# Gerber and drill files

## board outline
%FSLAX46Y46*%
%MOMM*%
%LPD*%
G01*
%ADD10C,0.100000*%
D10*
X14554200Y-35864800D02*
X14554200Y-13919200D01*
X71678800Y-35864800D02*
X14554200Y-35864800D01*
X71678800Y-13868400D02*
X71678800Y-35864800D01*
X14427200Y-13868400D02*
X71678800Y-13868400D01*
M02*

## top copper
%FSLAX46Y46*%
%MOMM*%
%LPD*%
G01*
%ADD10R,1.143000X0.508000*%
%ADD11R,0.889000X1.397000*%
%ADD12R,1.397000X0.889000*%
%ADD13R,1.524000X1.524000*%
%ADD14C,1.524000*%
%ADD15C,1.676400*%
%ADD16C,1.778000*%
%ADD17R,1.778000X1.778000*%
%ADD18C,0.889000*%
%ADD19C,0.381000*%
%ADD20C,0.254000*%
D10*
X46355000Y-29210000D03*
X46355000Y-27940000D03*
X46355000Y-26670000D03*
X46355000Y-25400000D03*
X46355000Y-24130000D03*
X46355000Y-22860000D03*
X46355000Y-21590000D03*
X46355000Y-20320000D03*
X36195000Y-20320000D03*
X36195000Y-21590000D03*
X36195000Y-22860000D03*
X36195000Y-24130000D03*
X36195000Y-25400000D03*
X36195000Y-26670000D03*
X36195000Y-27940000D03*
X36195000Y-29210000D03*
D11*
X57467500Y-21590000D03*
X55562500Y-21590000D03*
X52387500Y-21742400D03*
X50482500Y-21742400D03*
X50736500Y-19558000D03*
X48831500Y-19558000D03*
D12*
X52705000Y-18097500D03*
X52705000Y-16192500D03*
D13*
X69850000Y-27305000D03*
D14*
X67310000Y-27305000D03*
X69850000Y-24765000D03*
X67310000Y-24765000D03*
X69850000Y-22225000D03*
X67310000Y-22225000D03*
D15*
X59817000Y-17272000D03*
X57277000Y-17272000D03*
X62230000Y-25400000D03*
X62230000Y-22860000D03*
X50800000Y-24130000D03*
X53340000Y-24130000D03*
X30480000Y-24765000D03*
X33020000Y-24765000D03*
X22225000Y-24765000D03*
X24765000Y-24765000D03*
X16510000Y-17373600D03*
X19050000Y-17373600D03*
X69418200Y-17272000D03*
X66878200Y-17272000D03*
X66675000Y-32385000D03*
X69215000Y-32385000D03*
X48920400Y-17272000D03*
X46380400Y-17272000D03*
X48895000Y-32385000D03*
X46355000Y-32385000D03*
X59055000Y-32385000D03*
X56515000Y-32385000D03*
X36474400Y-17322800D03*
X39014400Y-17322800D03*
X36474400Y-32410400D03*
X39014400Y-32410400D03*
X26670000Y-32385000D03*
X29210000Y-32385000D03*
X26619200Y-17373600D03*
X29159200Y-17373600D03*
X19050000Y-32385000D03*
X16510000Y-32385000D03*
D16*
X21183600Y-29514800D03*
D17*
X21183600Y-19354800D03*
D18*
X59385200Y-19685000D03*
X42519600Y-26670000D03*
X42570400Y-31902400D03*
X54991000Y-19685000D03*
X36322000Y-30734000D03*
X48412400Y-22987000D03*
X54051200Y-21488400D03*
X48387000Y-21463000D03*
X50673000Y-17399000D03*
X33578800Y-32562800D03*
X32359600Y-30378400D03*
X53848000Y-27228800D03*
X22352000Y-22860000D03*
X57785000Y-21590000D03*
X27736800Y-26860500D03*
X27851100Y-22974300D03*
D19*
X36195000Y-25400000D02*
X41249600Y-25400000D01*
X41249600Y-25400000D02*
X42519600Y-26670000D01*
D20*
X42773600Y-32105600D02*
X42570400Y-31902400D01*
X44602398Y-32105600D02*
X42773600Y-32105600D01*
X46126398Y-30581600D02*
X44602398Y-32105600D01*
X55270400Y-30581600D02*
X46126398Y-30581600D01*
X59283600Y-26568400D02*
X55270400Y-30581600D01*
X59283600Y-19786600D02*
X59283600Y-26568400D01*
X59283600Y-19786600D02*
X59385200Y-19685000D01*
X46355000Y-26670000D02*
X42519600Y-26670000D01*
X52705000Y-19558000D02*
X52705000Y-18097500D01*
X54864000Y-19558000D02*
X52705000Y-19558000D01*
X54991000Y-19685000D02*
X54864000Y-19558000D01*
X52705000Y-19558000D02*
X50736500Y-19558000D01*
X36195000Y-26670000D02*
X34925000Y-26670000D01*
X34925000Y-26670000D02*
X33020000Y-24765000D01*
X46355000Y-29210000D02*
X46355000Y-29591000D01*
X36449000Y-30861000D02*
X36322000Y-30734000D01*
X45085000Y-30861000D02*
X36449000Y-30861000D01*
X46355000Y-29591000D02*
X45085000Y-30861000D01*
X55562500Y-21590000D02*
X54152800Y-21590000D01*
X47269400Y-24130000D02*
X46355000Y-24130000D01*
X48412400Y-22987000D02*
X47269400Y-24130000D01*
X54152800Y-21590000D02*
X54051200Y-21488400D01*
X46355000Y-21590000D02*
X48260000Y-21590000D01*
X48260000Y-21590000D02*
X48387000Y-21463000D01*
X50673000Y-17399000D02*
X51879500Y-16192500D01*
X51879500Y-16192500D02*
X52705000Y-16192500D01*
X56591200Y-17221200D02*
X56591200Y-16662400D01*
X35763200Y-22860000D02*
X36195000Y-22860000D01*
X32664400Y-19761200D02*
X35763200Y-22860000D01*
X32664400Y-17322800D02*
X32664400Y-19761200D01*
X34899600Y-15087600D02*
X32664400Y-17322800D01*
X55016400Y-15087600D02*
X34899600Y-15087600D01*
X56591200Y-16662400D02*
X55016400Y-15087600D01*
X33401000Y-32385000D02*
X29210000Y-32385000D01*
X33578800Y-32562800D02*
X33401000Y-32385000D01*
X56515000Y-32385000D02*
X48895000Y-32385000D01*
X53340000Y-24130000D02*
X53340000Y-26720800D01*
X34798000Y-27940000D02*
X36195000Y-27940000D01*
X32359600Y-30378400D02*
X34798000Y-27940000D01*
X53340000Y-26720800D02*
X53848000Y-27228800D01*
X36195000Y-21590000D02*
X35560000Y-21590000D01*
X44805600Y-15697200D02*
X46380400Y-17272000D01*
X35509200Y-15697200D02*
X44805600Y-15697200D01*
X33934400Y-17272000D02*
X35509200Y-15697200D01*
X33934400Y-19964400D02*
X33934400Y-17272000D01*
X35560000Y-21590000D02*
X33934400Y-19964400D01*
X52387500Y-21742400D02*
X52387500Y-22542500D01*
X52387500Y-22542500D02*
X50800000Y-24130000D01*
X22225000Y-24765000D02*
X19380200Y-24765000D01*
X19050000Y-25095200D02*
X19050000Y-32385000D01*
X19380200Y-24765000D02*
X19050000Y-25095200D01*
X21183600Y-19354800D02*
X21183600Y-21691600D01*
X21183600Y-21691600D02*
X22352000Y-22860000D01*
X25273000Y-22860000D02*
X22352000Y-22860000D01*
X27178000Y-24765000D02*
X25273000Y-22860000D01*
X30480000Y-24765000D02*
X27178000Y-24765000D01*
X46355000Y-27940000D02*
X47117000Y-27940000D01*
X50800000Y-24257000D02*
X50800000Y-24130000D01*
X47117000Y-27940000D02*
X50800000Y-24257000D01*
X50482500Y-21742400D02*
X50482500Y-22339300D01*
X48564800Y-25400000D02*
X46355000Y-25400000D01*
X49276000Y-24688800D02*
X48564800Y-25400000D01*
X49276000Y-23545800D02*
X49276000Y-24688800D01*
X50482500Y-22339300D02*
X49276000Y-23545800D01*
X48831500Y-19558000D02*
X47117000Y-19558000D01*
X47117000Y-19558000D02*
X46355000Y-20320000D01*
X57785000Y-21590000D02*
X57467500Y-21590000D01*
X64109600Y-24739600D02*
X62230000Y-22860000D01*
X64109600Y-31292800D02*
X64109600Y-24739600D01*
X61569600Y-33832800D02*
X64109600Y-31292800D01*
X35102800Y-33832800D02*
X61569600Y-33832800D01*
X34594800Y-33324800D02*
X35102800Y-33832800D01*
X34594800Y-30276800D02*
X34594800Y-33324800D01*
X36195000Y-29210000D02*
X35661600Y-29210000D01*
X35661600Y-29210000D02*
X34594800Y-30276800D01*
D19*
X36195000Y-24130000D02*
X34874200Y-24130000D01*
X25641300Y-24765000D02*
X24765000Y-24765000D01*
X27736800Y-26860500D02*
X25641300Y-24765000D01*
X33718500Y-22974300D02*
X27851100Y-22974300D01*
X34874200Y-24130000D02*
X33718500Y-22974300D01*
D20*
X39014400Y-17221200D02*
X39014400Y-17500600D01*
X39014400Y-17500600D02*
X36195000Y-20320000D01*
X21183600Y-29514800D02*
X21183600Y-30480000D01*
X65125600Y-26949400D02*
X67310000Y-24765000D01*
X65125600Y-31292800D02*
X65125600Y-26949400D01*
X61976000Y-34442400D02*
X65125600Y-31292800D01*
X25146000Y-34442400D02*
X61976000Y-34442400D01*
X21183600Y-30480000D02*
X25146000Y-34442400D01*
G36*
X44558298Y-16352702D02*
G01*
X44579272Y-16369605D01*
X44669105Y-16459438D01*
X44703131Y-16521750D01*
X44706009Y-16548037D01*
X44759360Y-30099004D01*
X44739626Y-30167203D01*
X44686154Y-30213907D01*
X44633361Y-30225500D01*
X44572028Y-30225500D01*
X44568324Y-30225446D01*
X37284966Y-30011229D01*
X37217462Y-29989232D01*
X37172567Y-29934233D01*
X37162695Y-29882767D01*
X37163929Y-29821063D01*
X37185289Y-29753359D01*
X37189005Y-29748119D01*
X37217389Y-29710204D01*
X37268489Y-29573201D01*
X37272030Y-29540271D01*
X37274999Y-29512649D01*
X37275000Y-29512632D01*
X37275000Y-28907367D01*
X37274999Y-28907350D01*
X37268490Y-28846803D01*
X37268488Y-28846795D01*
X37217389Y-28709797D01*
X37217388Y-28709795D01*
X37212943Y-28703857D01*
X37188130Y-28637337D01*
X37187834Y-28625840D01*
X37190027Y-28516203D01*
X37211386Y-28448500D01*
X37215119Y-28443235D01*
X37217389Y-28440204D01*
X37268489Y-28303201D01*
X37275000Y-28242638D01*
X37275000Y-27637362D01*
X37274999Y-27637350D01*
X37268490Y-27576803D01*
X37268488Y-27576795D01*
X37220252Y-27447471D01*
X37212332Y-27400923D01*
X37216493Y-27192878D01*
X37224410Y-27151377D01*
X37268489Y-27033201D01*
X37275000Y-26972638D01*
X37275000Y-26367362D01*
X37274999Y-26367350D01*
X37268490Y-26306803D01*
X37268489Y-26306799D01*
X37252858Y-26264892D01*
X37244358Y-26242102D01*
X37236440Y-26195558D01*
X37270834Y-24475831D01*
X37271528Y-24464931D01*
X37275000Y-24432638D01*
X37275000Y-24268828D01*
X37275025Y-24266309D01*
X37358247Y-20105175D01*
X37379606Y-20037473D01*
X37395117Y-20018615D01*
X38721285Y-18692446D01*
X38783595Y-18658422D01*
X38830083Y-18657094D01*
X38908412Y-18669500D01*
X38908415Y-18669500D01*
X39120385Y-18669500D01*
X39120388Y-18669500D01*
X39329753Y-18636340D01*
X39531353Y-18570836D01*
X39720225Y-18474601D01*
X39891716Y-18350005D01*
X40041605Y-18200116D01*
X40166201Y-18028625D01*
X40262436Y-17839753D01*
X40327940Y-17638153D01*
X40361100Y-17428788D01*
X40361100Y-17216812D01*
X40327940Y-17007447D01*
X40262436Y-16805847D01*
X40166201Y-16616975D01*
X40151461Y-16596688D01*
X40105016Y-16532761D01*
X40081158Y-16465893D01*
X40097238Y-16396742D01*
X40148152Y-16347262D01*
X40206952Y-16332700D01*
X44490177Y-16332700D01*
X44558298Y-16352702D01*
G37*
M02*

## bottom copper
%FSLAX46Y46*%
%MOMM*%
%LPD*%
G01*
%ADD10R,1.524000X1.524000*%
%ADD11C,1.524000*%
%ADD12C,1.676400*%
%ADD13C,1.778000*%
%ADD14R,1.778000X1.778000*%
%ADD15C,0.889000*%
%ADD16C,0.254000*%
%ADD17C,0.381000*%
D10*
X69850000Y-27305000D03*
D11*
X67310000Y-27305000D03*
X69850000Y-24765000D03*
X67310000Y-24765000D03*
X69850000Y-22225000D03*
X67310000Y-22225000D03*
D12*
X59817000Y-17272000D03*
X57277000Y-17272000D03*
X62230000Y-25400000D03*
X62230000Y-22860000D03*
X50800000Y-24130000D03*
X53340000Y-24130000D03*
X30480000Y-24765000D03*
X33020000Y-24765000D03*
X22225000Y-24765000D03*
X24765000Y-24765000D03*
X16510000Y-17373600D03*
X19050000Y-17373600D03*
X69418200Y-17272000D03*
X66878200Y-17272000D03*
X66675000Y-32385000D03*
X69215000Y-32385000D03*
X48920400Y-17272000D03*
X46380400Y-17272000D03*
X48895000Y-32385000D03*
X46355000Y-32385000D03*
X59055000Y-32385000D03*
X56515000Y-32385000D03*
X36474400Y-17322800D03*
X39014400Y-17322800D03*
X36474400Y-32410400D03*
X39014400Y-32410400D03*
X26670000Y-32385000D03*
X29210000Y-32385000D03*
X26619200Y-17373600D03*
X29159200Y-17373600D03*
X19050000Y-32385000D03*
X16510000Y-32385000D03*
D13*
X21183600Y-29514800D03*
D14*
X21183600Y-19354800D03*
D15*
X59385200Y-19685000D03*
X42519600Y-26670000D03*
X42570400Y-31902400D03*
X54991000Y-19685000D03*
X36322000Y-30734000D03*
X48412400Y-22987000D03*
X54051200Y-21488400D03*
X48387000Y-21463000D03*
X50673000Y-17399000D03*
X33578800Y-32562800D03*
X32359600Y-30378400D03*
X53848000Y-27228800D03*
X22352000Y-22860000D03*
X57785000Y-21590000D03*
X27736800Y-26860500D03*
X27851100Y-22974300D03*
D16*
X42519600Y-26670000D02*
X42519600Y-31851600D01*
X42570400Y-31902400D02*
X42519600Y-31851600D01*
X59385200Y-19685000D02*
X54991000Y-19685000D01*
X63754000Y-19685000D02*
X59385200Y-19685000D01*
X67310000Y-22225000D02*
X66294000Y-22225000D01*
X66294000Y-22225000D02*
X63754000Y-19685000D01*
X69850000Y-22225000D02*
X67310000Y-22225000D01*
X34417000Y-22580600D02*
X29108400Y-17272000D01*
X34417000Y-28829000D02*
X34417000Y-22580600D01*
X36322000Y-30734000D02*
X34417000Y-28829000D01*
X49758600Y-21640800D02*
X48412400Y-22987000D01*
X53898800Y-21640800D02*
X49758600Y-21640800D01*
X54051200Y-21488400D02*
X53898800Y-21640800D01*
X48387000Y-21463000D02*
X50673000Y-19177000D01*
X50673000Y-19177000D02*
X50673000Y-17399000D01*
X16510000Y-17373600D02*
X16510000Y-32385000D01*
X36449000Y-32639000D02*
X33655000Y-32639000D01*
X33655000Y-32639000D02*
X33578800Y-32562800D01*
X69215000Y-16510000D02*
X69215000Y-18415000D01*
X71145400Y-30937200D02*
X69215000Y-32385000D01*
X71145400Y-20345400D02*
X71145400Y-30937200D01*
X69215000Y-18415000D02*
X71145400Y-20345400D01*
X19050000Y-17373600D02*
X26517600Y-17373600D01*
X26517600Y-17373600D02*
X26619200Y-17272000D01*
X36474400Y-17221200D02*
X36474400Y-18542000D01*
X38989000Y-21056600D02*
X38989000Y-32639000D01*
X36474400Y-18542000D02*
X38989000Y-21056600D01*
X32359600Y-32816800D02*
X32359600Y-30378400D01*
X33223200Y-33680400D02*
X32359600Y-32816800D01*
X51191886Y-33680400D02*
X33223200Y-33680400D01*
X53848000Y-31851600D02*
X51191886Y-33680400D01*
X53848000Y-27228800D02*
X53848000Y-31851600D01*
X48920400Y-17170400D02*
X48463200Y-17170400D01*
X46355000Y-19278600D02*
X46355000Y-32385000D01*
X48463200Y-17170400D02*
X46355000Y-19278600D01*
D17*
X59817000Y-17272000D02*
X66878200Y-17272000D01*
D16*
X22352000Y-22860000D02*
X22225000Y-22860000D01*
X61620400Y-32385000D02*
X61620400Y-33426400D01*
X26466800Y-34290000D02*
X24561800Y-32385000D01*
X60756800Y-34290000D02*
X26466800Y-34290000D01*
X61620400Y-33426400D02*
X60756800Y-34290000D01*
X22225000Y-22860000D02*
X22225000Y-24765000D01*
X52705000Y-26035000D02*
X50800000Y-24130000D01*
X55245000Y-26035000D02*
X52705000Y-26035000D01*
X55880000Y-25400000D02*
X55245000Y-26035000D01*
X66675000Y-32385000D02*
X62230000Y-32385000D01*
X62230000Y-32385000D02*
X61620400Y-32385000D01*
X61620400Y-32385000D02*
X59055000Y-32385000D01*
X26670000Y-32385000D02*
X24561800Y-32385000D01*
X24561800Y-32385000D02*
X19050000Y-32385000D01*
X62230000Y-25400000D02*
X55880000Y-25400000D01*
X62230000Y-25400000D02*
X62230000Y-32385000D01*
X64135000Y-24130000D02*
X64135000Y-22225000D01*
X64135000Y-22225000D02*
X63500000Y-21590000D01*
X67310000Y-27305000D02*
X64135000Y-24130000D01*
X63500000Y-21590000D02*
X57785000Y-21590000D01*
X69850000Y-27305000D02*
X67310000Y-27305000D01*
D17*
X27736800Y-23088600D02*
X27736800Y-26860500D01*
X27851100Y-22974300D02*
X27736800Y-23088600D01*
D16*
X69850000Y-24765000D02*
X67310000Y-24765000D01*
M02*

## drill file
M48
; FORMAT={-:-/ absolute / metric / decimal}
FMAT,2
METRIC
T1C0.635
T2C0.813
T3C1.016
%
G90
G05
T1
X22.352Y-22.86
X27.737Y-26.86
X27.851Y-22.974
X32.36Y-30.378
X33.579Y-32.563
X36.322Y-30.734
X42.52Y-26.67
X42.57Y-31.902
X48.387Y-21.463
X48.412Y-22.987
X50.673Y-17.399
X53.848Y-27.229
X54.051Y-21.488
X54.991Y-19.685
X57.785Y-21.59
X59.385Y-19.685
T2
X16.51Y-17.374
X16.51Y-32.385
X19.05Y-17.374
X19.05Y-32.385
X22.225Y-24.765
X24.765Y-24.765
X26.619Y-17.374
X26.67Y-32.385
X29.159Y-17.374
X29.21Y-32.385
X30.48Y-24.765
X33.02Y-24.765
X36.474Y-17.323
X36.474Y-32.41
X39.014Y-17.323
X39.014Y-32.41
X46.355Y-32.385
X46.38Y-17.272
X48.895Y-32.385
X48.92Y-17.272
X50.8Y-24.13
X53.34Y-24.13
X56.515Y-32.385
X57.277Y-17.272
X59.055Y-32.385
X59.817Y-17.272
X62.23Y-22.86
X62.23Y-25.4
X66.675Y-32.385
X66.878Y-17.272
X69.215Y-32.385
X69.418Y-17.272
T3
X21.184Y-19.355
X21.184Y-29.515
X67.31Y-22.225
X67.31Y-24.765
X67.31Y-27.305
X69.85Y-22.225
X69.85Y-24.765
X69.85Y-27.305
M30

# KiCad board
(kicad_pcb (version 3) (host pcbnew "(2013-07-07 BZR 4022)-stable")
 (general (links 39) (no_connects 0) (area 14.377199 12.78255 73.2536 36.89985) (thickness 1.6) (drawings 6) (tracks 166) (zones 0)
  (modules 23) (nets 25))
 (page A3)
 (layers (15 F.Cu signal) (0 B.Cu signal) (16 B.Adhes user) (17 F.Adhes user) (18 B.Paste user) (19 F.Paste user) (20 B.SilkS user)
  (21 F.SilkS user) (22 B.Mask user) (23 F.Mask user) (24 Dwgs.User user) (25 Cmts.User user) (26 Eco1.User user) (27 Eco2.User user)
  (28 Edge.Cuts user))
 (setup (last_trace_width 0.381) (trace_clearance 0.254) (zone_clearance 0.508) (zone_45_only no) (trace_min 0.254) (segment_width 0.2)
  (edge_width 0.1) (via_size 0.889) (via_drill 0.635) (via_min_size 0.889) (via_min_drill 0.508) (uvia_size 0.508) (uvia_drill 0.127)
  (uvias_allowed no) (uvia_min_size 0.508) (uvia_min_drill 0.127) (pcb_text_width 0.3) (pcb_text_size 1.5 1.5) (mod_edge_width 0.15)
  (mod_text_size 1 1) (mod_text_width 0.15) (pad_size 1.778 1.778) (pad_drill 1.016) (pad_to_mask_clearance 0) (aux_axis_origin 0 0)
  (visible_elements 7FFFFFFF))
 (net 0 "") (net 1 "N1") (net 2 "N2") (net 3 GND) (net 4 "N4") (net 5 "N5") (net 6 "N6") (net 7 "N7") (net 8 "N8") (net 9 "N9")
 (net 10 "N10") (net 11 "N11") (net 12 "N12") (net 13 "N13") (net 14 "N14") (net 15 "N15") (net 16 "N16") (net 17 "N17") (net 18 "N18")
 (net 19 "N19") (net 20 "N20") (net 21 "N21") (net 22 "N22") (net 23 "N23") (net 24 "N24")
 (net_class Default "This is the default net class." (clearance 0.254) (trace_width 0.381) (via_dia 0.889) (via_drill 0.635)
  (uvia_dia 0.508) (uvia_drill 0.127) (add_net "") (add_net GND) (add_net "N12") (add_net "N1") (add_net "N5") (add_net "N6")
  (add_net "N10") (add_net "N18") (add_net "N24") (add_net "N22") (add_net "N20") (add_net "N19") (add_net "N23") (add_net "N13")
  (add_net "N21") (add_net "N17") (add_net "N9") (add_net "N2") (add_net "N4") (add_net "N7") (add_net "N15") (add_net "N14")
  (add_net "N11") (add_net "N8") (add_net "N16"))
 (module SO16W (layer F.Cu) (at 41.275 24.765 90)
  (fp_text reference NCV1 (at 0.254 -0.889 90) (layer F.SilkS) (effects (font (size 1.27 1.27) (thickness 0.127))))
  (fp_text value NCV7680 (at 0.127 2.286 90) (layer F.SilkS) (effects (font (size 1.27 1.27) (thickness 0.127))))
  (pad 1 smd rect (at -4.445 5.08 90) (size 0.508 1.143) (layers F.Cu F.Paste F.Mask) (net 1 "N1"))
  (pad 2 smd rect (at -3.175 5.08 90) (size 0.508 1.143) (layers F.Cu F.Paste F.Mask) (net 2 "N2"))
  (pad 3 smd rect (at -1.905 5.08 90) (size 0.508 1.143) (layers F.Cu F.Paste F.Mask) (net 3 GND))
  (pad 4 smd rect (at -0.635 5.08 90) (size 0.508 1.143) (layers F.Cu F.Paste F.Mask) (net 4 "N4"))
  (pad 5 smd rect (at 0.635 5.08 90) (size 0.508 1.143) (layers F.Cu F.Paste F.Mask) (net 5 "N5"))
  (pad 6 smd rect (at 1.905 5.08 90) (size 0.508 1.143) (layers F.Cu F.Paste F.Mask))
  (pad 7 smd rect (at 3.175 5.08 90) (size 0.508 1.143) (layers F.Cu F.Paste F.Mask) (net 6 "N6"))
  (pad 8 smd rect (at 4.445 5.08 90) (size 0.508 1.143) (layers F.Cu F.Paste F.Mask) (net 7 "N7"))
  (pad 9 smd rect (at 4.445 -5.08 90) (size 0.508 1.143) (layers F.Cu F.Paste F.Mask) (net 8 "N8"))
  (pad 10 smd rect (at 3.175 -5.08 90) (size 0.508 1.143) (layers F.Cu F.Paste F.Mask) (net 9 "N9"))
  (pad 11 smd rect (at 1.905 -5.08 90) (size 0.508 1.143) (layers F.Cu F.Paste F.Mask) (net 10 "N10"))
  (pad 12 smd rect (at 0.635 -5.08 90) (size 0.508 1.143) (layers F.Cu F.Paste F.Mask) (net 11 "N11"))
  (pad 13 smd rect (at -0.635 -5.08 90) (size 0.508 1.143) (layers F.Cu F.Paste F.Mask) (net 3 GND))
  (pad 14 smd rect (at -1.905 -5.08 90) (size 0.508 1.143) (layers F.Cu F.Paste F.Mask) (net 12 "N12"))
  (pad 15 smd rect (at -3.175 -5.08 90) (size 0.508 1.143) (layers F.Cu F.Paste F.Mask) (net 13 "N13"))
  (pad 16 smd rect (at -4.445 -5.08 90) (size 0.508 1.143) (layers F.Cu F.Paste F.Mask) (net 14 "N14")))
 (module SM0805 (layer F.Cu) (at 56.515 21.59 180)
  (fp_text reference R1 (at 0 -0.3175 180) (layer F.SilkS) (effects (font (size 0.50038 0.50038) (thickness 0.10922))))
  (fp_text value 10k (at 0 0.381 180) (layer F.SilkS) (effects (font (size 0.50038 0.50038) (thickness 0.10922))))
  (pad 1 smd rect (at -0.9525 0 180) (size 0.889 1.397) (layers F.Cu F.Paste F.Mask) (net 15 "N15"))
  (pad 2 smd rect (at 0.9525 0 180) (size 0.889 1.397) (layers F.Cu F.Paste F.Mask) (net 5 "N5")))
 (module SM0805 (layer F.Cu) (at 51.435 21.7424 180)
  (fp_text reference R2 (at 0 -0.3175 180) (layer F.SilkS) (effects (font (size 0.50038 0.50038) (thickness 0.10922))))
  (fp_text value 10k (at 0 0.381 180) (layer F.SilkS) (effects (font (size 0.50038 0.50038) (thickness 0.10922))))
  (pad 1 smd rect (at -0.9525 0 180) (size 0.889 1.397) (layers F.Cu F.Paste F.Mask) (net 2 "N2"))
  (pad 2 smd rect (at 0.9525 0 180) (size 0.889 1.397) (layers F.Cu F.Paste F.Mask) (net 4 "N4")))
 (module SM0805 (layer F.Cu) (at 49.784 19.558 180)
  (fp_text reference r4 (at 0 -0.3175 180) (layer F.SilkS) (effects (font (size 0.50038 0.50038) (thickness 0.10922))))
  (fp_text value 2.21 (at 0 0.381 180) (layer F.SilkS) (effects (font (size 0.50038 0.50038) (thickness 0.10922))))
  (pad 1 smd rect (at -0.9525 0 180) (size 0.889 1.397) (layers F.Cu F.Paste F.Mask) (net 3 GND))
  (pad 2 smd rect (at 0.9525 0 180) (size 0.889 1.397) (layers F.Cu F.Paste F.Mask) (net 7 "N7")))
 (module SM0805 (layer F.Cu) (at 52.705 17.145 90)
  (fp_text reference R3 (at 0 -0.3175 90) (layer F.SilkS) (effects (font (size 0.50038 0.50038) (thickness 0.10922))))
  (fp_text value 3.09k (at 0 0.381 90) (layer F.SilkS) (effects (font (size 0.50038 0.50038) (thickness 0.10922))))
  (pad 1 smd rect (at -0.9525 0 90) (size 0.889 1.397) (layers F.Cu F.Paste F.Mask) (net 3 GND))
  (pad 2 smd rect (at 0.9525 0 90) (size 0.889 1.397) (layers F.Cu F.Paste F.Mask) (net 6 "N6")))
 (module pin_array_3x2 (layer F.Cu) (at 68.58 24.765 90)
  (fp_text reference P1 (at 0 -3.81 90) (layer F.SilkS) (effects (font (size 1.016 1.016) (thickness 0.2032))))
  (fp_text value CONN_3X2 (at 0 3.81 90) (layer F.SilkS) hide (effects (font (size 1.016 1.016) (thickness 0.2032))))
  (pad 1 thru_hole rect (at -2.54 1.27 90) (size 1.524 1.524) (drill 1.016) (layers *.Cu *.Mask F.SilkS) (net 15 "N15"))
  (pad 2 thru_hole circle (at -2.54 -1.27 90) (size 1.524 1.524) (drill 1.016) (layers *.Cu *.Mask F.SilkS) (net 15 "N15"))
  (pad 3 thru_hole circle (at 0 1.27 90) (size 1.524 1.524) (drill 1.016) (layers *.Cu *.Mask F.SilkS) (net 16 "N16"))
  (pad 4 thru_hole circle (at 0 -1.27 90) (size 1.524 1.524) (drill 1.016) (layers *.Cu *.Mask F.SilkS) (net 16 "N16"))
  (pad 5 thru_hole circle (at 2.54 1.27 90) (size 1.524 1.524) (drill 1.016) (layers *.Cu *.Mask F.SilkS) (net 3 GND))
  (pad 6 thru_hole circle (at 2.54 -1.27 90) (size 1.524 1.524) (drill 1.016) (layers *.Cu *.Mask F.SilkS) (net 3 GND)))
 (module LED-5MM (layer B.Cu) (at 58.547 17.272 180)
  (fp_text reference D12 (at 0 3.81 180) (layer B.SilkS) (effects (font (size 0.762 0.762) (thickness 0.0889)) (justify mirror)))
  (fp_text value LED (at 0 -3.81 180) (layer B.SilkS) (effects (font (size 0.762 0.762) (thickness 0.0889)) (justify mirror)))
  (pad 1 thru_hole circle (at -1.27 0 180) (size 1.6764 1.6764) (drill 0.8128) (layers *.Cu *.Mask B.SilkS) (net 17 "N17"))
  (pad 2 thru_hole circle (at 1.27 0 180) (size 1.6764 1.6764) (drill 0.8128) (layers *.Cu *.Mask B.SilkS) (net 10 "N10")))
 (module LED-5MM (layer B.Cu) (at 62.23 24.13 90)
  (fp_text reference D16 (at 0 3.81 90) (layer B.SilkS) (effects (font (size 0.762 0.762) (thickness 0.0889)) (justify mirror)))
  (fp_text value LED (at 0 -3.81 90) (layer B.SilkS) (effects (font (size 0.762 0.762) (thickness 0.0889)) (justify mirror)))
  (pad 1 thru_hole circle (at -1.27 0 90) (size 1.6764 1.6764) (drill 0.8128) (layers *.Cu *.Mask B.SilkS) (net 2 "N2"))
  (pad 2 thru_hole circle (at 1.27 0 90) (size 1.6764 1.6764) (drill 0.8128) (layers *.Cu *.Mask B.SilkS) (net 14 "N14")))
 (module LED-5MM (layer B.Cu) (at 52.07 24.13)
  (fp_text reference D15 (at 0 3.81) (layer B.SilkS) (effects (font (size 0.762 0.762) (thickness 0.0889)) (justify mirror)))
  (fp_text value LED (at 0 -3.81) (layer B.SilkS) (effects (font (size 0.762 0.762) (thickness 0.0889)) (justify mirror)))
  (pad 1 thru_hole circle (at -1.27 0) (size 1.6764 1.6764) (drill 0.8128) (layers *.Cu *.Mask B.SilkS) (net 2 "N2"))
  (pad 2 thru_hole circle (at 1.27 0) (size 1.6764 1.6764) (drill 0.8128) (layers *.Cu *.Mask B.SilkS) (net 13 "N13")))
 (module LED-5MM (layer B.Cu) (at 31.75 24.765)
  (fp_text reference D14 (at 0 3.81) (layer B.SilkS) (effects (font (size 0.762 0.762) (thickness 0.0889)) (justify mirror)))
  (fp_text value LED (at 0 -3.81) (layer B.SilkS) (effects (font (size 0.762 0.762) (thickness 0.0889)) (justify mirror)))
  (pad 1 thru_hole circle (at -1.27 0) (size 1.6764 1.6764) (drill 0.8128) (layers *.Cu *.Mask B.SilkS) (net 2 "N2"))
  (pad 2 thru_hole circle (at 1.27 0) (size 1.6764 1.6764) (drill 0.8128) (layers *.Cu *.Mask B.SilkS) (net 12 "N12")))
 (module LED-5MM (layer B.Cu) (at 23.495 24.765)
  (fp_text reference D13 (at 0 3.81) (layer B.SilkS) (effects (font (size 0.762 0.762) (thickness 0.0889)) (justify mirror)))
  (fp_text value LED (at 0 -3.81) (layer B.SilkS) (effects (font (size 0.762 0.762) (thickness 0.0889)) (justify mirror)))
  (pad 1 thru_hole circle (at -1.27 0) (size 1.6764 1.6764) (drill 0.8128) (layers *.Cu *.Mask B.SilkS) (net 2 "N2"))
  (pad 2 thru_hole circle (at 1.27 0) (size 1.6764 1.6764) (drill 0.8128) (layers *.Cu *.Mask B.SilkS) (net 11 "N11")))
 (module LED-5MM (layer B.Cu) (at 17.78 17.3736)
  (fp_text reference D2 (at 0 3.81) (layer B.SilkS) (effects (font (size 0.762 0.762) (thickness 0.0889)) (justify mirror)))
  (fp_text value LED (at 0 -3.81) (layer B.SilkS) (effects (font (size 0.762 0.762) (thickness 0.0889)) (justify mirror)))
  (pad 1 thru_hole circle (at -1.27 0) (size 1.6764 1.6764) (drill 0.8128) (layers *.Cu *.Mask B.SilkS) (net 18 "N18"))
  (pad 2 thru_hole circle (at 1.27 0) (size 1.6764 1.6764) (drill 0.8128) (layers *.Cu *.Mask B.SilkS) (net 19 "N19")))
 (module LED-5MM (layer B.Cu) (at 68.1482 17.272 180)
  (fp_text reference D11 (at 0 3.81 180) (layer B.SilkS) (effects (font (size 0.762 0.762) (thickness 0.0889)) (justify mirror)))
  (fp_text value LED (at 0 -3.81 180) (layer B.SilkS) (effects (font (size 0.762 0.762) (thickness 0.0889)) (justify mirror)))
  (pad 1 thru_hole circle (at -1.27 0 180) (size 1.6764 1.6764) (drill 0.8128) (layers *.Cu *.Mask B.SilkS) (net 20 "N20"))
  (pad 2 thru_hole circle (at 1.27 0 180) (size 1.6764 1.6764) (drill 0.8128) (layers *.Cu *.Mask B.SilkS) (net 17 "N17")))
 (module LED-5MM (layer B.Cu) (at 67.945 32.385)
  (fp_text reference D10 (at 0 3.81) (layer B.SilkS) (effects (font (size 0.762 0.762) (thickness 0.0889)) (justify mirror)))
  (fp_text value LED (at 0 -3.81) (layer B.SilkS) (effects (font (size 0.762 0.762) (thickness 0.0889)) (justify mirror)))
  (pad 1 thru_hole circle (at -1.27 0) (size 1.6764 1.6764) (drill 0.8128) (layers *.Cu *.Mask B.SilkS) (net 2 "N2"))
  (pad 2 thru_hole circle (at 1.27 0) (size 1.6764 1.6764) (drill 0.8128) (layers *.Cu *.Mask B.SilkS) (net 20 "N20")))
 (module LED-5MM (layer B.Cu) (at 47.6504 17.272 180)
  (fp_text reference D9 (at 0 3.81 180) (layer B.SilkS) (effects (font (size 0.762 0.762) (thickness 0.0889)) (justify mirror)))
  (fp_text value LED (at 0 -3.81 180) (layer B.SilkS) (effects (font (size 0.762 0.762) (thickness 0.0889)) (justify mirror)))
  (pad 1 thru_hole circle (at -1.27 0 180) (size 1.6764 1.6764) (drill 0.8128) (layers *.Cu *.Mask B.SilkS) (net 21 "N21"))
  (pad 2 thru_hole circle (at 1.27 0 180) (size 1.6764 1.6764) (drill 0.8128) (layers *.Cu *.Mask B.SilkS) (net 9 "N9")))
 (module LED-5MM (layer B.Cu) (at 47.625 32.385 180)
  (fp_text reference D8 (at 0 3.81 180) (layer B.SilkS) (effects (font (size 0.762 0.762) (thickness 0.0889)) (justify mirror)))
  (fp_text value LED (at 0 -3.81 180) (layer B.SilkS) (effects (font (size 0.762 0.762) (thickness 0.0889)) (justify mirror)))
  (pad 1 thru_hole circle (at -1.27 0 180) (size 1.6764 1.6764) (drill 0.8128) (layers *.Cu *.Mask B.SilkS) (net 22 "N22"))
  (pad 2 thru_hole circle (at 1.27 0 180) (size 1.6764 1.6764) (drill 0.8128) (layers *.Cu *.Mask B.SilkS) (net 21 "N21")))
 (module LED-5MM (layer B.Cu) (at 57.785 32.385 180)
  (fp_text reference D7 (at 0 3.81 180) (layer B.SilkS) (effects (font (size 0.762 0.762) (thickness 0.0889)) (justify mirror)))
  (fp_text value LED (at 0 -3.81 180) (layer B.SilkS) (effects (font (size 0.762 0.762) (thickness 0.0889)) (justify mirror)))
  (pad 1 thru_hole circle (at -1.27 0 180) (size 1.6764 1.6764) (drill 0.8128) (layers *.Cu *.Mask B.SilkS) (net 2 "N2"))
  (pad 2 thru_hole circle (at 1.27 0 180) (size 1.6764 1.6764) (drill 0.8128) (layers *.Cu *.Mask B.SilkS) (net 22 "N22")))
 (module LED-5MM (layer B.Cu) (at 37.7444 17.3228)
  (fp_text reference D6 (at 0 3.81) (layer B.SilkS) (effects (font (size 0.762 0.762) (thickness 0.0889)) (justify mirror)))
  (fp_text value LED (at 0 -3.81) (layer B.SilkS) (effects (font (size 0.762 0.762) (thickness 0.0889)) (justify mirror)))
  (pad 1 thru_hole circle (at -1.27 0) (size 1.6764 1.6764) (drill 0.8128) (layers *.Cu *.Mask B.SilkS) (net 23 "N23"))
  (pad 2 thru_hole circle (at 1.27 0) (size 1.6764 1.6764) (drill 0.8128) (layers *.Cu *.Mask B.SilkS) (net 8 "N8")))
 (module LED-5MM (layer B.Cu) (at 37.7444 32.4104)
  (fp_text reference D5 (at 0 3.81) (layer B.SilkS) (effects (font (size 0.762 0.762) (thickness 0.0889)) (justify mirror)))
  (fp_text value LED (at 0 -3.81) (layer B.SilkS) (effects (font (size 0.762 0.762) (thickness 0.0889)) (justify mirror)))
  (pad 1 thru_hole circle (at -1.27 0) (size 1.6764 1.6764) (drill 0.8128) (layers *.Cu *.Mask B.SilkS) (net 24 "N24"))
  (pad 2 thru_hole circle (at 1.27 0) (size 1.6764 1.6764) (drill 0.8128) (layers *.Cu *.Mask B.SilkS) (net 23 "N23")))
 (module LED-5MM (layer B.Cu) (at 27.94 32.385)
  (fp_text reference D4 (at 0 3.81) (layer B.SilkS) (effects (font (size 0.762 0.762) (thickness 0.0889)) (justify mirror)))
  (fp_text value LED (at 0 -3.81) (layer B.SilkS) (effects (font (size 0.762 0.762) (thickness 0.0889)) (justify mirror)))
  (pad 1 thru_hole circle (at -1.27 0) (size 1.6764 1.6764) (drill 0.8128) (layers *.Cu *.Mask B.SilkS) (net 2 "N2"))
  (pad 2 thru_hole circle (at 1.27 0) (size 1.6764 1.6764) (drill 0.8128) (layers *.Cu *.Mask B.SilkS) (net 24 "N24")))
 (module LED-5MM (layer B.Cu) (at 27.8892 17.3736)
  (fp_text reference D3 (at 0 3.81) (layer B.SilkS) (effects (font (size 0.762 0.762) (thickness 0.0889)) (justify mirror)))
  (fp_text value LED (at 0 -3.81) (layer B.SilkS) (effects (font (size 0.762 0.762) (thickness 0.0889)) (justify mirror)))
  (pad 1 thru_hole circle (at -1.27 0) (size 1.6764 1.6764) (drill 0.8128) (layers *.Cu *.Mask B.SilkS) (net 19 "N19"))
  (pad 2 thru_hole circle (at 1.27 0) (size 1.6764 1.6764) (drill 0.8128) (layers *.Cu *.Mask B.SilkS) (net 1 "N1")))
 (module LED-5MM (layer B.Cu) (at 17.78 32.385 180)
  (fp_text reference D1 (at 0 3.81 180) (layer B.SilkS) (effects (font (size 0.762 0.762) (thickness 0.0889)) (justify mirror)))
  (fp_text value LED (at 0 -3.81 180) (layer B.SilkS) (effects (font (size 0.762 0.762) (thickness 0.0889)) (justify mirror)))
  (pad 1 thru_hole circle (at -1.27 0 180) (size 1.6764 1.6764) (drill 0.8128) (layers *.Cu *.Mask B.SilkS) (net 2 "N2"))
  (pad 2 thru_hole circle (at 1.27 0 180) (size 1.6764 1.6764) (drill 0.8128) (layers *.Cu *.Mask B.SilkS) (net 18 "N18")))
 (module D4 (layer F.Cu) (at 21.1836 24.4348 90)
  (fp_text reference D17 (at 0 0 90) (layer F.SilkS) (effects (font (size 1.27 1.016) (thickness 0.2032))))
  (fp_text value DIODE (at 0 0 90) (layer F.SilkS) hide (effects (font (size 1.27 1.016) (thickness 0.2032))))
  (pad 1 thru_hole circle (at -5.08 0 90) (size 1.778 1.778) (drill 1.016) (layers *.Cu *.Mask F.SilkS) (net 16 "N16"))
  (pad 2 thru_hole rect (at 5.08 0 90) (size 1.778 1.778) (drill 1.016) (layers *.Cu *.Mask F.SilkS) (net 2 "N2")))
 (gr_line (start 14.5542 35.8648) (end 14.5542 13.9192) (angle 90) (layer Edge.Cuts) (width 0.1))
 (gr_line (start 71.6788 35.8648) (end 14.5542 35.8648) (angle 90) (layer Edge.Cuts) (width 0.1))
 (gr_line (start 71.6788 13.8684) (end 71.6788 35.8648) (angle 90) (layer Edge.Cuts) (width 0.1))
 (gr_line (start 14.4272 13.8684) (end 71.6788 13.8684) (angle 90) (layer Edge.Cuts) (width 0.1))
 (segment (start 36.195 25.4) (end 41.2496 25.4) (width 0.381) (layer F.Cu) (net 3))
 (segment (start 41.2496 25.4) (end 42.5196 26.67) (width 0.381) (layer F.Cu) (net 3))
 (via (at 59.3852 19.685) (size 0.889) (layers F.Cu B.Cu) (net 3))
 (via (at 42.5196 26.67) (size 0.889) (layers F.Cu B.Cu) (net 3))
 (segment (start 42.5196 26.67) (end 42.5196 31.8516) (width 0.254) (layer B.Cu) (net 3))
 (segment (start 42.5704 31.9024) (end 42.5196 31.8516) (width 0.254) (layer B.Cu) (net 3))
 (via (at 42.5704 31.9024) (size 0.889) (layers F.Cu B.Cu) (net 3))
 (segment (start 42.7736 32.1056) (end 42.5704 31.9024) (width 0.254) (layer F.Cu) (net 3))
 (segment (start 44.602398 32.1056) (end 42.7736 32.1056) (width 0.254) (layer F.Cu) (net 3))
 (segment (start 46.126398 30.5816) (end 44.602398 32.1056) (width 0.254) (layer F.Cu) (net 3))
 (segment (start 55.2704 30.5816) (end 46.126398 30.5816) (width 0.254) (layer F.Cu) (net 3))
 (segment (start 59.2836 26.5684) (end 55.2704 30.5816) (width 0.254) (layer F.Cu) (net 3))
 (segment (start 59.2836 19.7866) (end 59.2836 26.5684) (width 0.254) (layer F.Cu) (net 3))
 (segment (start 59.2836 19.7866) (end 59.3852 19.685) (width 0.254) (layer F.Cu) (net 3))
 (segment (start 46.355 26.67) (end 42.5196 26.67) (width 0.254) (layer F.Cu) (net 3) (status 10))
 (segment (start 52.705 19.558) (end 52.705 18.0975) (width 0.254) (layer F.Cu) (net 3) (status 20))
 (segment (start 54.864 19.558) (end 52.705 19.558) (width 0.254) (layer F.Cu) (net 3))
 (segment (start 59.3852 19.685) (end 54.991 19.685) (width 0.254) (layer B.Cu) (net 3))
 (via (at 54.991 19.685) (size 0.889) (layers F.Cu B.Cu) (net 3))
 (segment (start 54.991 19.685) (end 54.864 19.558) (width 0.254) (layer F.Cu) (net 3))
 (segment (start 52.705 19.558) (end 50.7365 19.558) (width 0.254) (layer F.Cu) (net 3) (status 20))
 (segment (start 63.754 19.685) (end 59.3852 19.685) (width 0.254) (layer B.Cu) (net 3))
 (segment (start 67.31 22.225) (end 66.294 22.225) (width 0.254) (layer B.Cu) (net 3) (status 10))
 (segment (start 66.294 22.225) (end 63.754 19.685) (width 0.254) (layer B.Cu) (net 3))
 (segment (start 69.85 22.225) (end 67.31 22.225) (width 0.254) (layer B.Cu) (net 3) (status 30))
 (segment (start 36.195 26.67) (end 34.925 26.67) (width 0.254) (layer F.Cu) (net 12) (status 10))
 (segment (start 34.925 26.67) (end 33.02 24.765) (width 0.254) (layer F.Cu) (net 12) (status 20))
 (segment (start 46.355 29.21) (end 46.355 29.591) (width 0.254) (layer F.Cu) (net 1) (status 10))
 (segment (start 34.417 22.5806) (end 29.1084 17.272) (width 0.254) (layer B.Cu) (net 1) (status 20))
 (segment (start 34.417 28.829) (end 34.417 22.5806) (width 0.254) (layer B.Cu) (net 1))
 (segment (start 36.322 30.734) (end 34.417 28.829) (width 0.254) (layer B.Cu) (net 1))
 (via (at 36.322 30.734) (size 0.889) (layers F.Cu B.Cu) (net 1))
 (segment (start 36.449 30.861) (end 36.322 30.734) (width 0.254) (layer F.Cu) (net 1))
 (segment (start 45.085 30.861) (end 36.449 30.861) (width 0.254) (layer F.Cu) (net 1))
 (segment (start 46.355 29.591) (end 45.085 30.861) (width 0.254) (layer F.Cu) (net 1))
 (segment (start 55.5625 21.59) (end 54.1528 21.59) (width 0.254) (layer F.Cu) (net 5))
 (segment (start 47.2694 24.13) (end 46.355 24.13) (width 0.254) (layer F.Cu) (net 5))
 (segment (start 48.4124 22.987) (end 47.2694 24.13) (width 0.254) (layer F.Cu) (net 5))
 (via (at 48.4124 22.987) (size 0.889) (layers F.Cu B.Cu) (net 5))
 (segment (start 49.7586 21.6408) (end 48.4124 22.987) (width 0.254) (layer B.Cu) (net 5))
 (segment (start 53.8988 21.6408) (end 49.7586 21.6408) (width 0.254) (layer B.Cu) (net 5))
 (segment (start 54.0512 21.4884) (end 53.8988 21.6408) (width 0.254) (layer B.Cu) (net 5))
 (via (at 54.0512 21.4884) (size 0.889) (layers F.Cu B.Cu) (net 5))
 (segment (start 54.1528 21.59) (end 54.0512 21.4884) (width 0.254) (layer F.Cu) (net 5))
 (segment (start 46.355 21.59) (end 48.26 21.59) (width 0.254) (layer F.Cu) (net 6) (status 10))
 (segment (start 48.26 21.59) (end 48.387 21.463) (width 0.254) (layer F.Cu) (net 6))
 (via (at 48.387 21.463) (size 0.889) (layers F.Cu B.Cu) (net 6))
 (segment (start 48.387 21.463) (end 50.673 19.177) (width 0.254) (layer B.Cu) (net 6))
 (segment (start 50.673 19.177) (end 50.673 17.399) (width 0.254) (layer B.Cu) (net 6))
 (via (at 50.673 17.399) (size 0.889) (layers F.Cu B.Cu) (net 6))
 (segment (start 50.673 17.399) (end 51.8795 16.1925) (width 0.254) (layer F.Cu) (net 6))
 (segment (start 51.8795 16.1925) (end 52.705 16.1925) (width 0.254) (layer F.Cu) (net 6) (status 20))
 (segment (start 56.5912 17.2212) (end 56.5912 16.6624) (width 0.254) (layer F.Cu) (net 10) (status 30))
 (segment (start 35.7632 22.86) (end 36.195 22.86) (width 0.254) (layer F.Cu) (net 10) (status 30))
 (segment (start 32.6644 19.7612) (end 35.7632 22.86) (width 0.254) (layer F.Cu) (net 10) (status 20))
 (segment (start 32.6644 17.3228) (end 32.6644 19.7612) (width 0.254) (layer F.Cu) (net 10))
 (segment (start 34.8996 15.0876) (end 32.6644 17.3228) (width 0.254) (layer F.Cu) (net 10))
 (segment (start 55.0164 15.0876) (end 34.8996 15.0876) (width 0.254) (layer F.Cu) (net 10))
 (segment (start 56.5912 16.6624) (end 55.0164 15.0876) (width 0.254) (layer F.Cu) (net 10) (status 10))
 (segment (start 16.51 17.3736) (end 16.51 32.385) (width 0.254) (layer B.Cu) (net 18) (status 30))
 (segment (start 36.449 32.639) (end 33.655 32.639) (width 0.254) (layer B.Cu) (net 24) (status 10))
 (segment (start 33.401 32.385) (end 29.21 32.385) (width 0.254) (layer F.Cu) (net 24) (status 20))
 (segment (start 33.5788 32.5628) (end 33.401 32.385) (width 0.254) (layer F.Cu) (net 24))
 (via (at 33.5788 32.5628) (size 0.889) (layers F.Cu B.Cu) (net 24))
 (segment (start 33.655 32.639) (end 33.5788 32.5628) (width 0.254) (layer B.Cu) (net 24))
 (segment (start 56.515 32.385) (end 48.895 32.385) (width 0.254) (layer F.Cu) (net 22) (status 30))
 (segment (start 69.215 16.51) (end 69.215 18.415) (width 0.254) (layer B.Cu) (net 20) (status 10))
 (segment (start 71.1454 30.9372) (end 69.215 32.385) (width 0.254) (layer B.Cu) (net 20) (status 20))
 (segment (start 71.1454 20.3454) (end 71.1454 30.9372) (width 0.254) (layer B.Cu) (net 20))
 (segment (start 69.215 18.415) (end 71.1454 20.3454) (width 0.254) (layer B.Cu) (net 20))
 (segment (start 19.05 17.3736) (end 26.5176 17.3736) (width 0.254) (layer B.Cu) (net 19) (status 30))
 (segment (start 26.5176 17.3736) (end 26.6192 17.272) (width 0.254) (layer B.Cu) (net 19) (status 30))
 (segment (start 36.4744 17.2212) (end 36.4744 18.542) (width 0.254) (layer B.Cu) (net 23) (status 10))
 (segment (start 38.989 21.0566) (end 38.989 32.639) (width 0.254) (layer B.Cu) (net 23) (status 20))
 (segment (start 36.4744 18.542) (end 38.989 21.0566) (width 0.254) (layer B.Cu) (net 23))
 (segment (start 53.34 24.13) (end 53.34 26.7208) (width 0.254) (layer F.Cu) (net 13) (status 10))
 (segment (start 34.798 27.94) (end 36.195 27.94) (width 0.254) (layer F.Cu) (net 13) (status 20))
 (segment (start 32.3596 30.3784) (end 34.798 27.94) (width 0.254) (layer F.Cu) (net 13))
 (via (at 32.3596 30.3784) (size 0.889) (layers F.Cu B.Cu) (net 13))
 (segment (start 32.3596 32.8168) (end 32.3596 30.3784) (width 0.254) (layer B.Cu) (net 13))
 (segment (start 33.2232 33.6804) (end 32.3596 32.8168) (width 0.254) (layer B.Cu) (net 13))
 (segment (start 51.191886 33.6804) (end 33.2232 33.6804) (width 0.254) (layer B.Cu) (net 13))
 (segment (start 53.848 31.8516) (end 51.191886 33.6804) (width 0.254) (layer B.Cu) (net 13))
 (segment (start 53.848 27.2288) (end 53.848 31.8516) (width 0.254) (layer B.Cu) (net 13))
 (via (at 53.848 27.2288) (size 0.889) (layers F.Cu B.Cu) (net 13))
 (segment (start 53.34 26.7208) (end 53.848 27.2288) (width 0.254) (layer F.Cu) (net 13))
 (segment (start 48.9204 17.1704) (end 48.4632 17.1704) (width 0.254) (layer B.Cu) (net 21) (status 30))
 (segment (start 46.355 19.2786) (end 46.355 32.385) (width 0.254) (layer B.Cu) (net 21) (status 20))
 (segment (start 48.4632 17.1704) (end 46.355 19.2786) (width 0.254) (layer B.Cu) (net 21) (status 10))
 (segment (start 59.817 17.272) (end 66.8782 17.272) (width 0.381) (layer B.Cu) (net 17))
 (segment (start 36.195 21.59) (end 35.56 21.59) (width 0.254) (layer F.Cu) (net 9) (status 10))
 (segment (start 44.8056 15.6972) (end 46.3804 17.272) (width 0.254) (layer F.Cu) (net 9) (status 20))
 (segment (start 35.5092 15.6972) (end 44.8056 15.6972) (width 0.254) (layer F.Cu) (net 9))
 (segment (start 33.9344 17.272) (end 35.5092 15.6972) (width 0.254) (layer F.Cu) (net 9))
 (segment (start 33.9344 19.9644) (end 33.9344 17.272) (width 0.254) (layer F.Cu) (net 9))
 (segment (start 35.56 21.59) (end 33.9344 19.9644) (width 0.254) (layer F.Cu) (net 9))
 (segment (start 52.3875 21.7424) (end 52.3875 22.5425) (width 0.254) (layer F.Cu) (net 2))
 (segment (start 52.3875 22.5425) (end 50.8 24.13) (width 0.254) (layer F.Cu) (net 2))
 (segment (start 22.225 24.765) (end 19.3802 24.765) (width 0.254) (layer F.Cu) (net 2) (status 10))
 (segment (start 19.05 25.0952) (end 19.05 32.385) (width 0.254) (layer F.Cu) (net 2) (status 20))
 (segment (start 19.3802 24.765) (end 19.05 25.0952) (width 0.254) (layer F.Cu) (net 2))
 (segment (start 21.1836 19.3548) (end 21.1836 21.6916) (width 0.254) (layer F.Cu) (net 2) (status 10))
 (segment (start 21.1836 21.6916) (end 22.352 22.86) (width 0.254) (layer F.Cu) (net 2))
 (segment (start 22.352 22.86) (end 22.225 22.86) (width 0.254) (layer B.Cu) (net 2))
 (via (at 22.352 22.86) (size 0.889) (layers F.Cu B.Cu) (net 2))
 (segment (start 25.273 22.86) (end 22.352 22.86) (width 0.254) (layer F.Cu) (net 2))
 (segment (start 27.178 24.765) (end 25.273 22.86) (width 0.254) (layer F.Cu) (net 2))
 (segment (start 61.6204 32.385) (end 61.6204 33.4264) (width 0.254) (layer B.Cu) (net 2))
 (segment (start 26.4668 34.29) (end 24.5618 32.385) (width 0.254) (layer B.Cu) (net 2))
 (segment (start 60.7568 34.29) (end 26.4668 34.29) (width 0.254) (layer B.Cu) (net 2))
 (segment (start 61.6204 33.4264) (end 60.7568 34.29) (width 0.254) (layer B.Cu) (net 2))
 (segment (start 30.48 24.765) (end 27.178 24.765) (width 0.254) (layer F.Cu) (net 2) (status 10))
 (segment (start 46.355 27.94) (end 47.117 27.94) (width 0.254) (layer F.Cu) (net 2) (status 10))
 (segment (start 50.8 24.257) (end 50.8 24.13) (width 0.254) (layer F.Cu) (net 2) (status 30))
 (segment (start 47.117 27.94) (end 50.8 24.257) (width 0.254) (layer F.Cu) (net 2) (status 20))
 (segment (start 22.225 22.86) (end 22.225 24.765) (width 0.254) (layer B.Cu) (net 2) (status 20))
 (segment (start 52.705 26.035) (end 50.8 24.13) (width 0.254) (layer B.Cu) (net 2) (status 20))
 (segment (start 55.245 26.035) (end 52.705 26.035) (width 0.254) (layer B.Cu) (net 2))
 (segment (start 55.88 25.4) (end 55.245 26.035) (width 0.254) (layer B.Cu) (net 2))
 (segment (start 66.675 32.385) (end 62.23 32.385) (width 0.254) (layer B.Cu) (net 2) (status 10))
 (segment (start 62.23 32.385) (end 61.6204 32.385) (width 0.254) (layer B.Cu) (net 2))
 (segment (start 61.6204 32.385) (end 59.055 32.385) (width 0.254) (layer B.Cu) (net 2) (status 20))
 (segment (start 26.67 32.385) (end 24.5618 32.385) (width 0.254) (layer B.Cu) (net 2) (status 10))
 (segment (start 24.5618 32.385) (end 19.05 32.385) (width 0.254) (layer B.Cu) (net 2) (status 20))
 (segment (start 62.23 25.4) (end 55.88 25.4) (width 0.254) (layer B.Cu) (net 2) (status 10))
 (segment (start 62.23 25.4) (end 62.23 32.385) (width 0.254) (layer B.Cu) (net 2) (status 10))
 (segment (start 50.4825 21.7424) (end 50.4825 22.3393) (width 0.254) (layer F.Cu) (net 4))
 (segment (start 48.5648 25.4) (end 46.355 25.4) (width 0.254) (layer F.Cu) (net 4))
 (segment (start 49.276 24.6888) (end 48.5648 25.4) (width 0.254) (layer F.Cu) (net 4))
 (segment (start 49.276 23.5458) (end 49.276 24.6888) (width 0.254) (layer F.Cu) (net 4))
 (segment (start 50.4825 22.3393) (end 49.276 23.5458) (width 0.254) (layer F.Cu) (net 4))
 (segment (start 48.8315 19.558) (end 47.117 19.558) (width 0.254) (layer F.Cu) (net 7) (status 10))
 (segment (start 47.117 19.558) (end 46.355 20.32) (width 0.254) (layer F.Cu) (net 7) (status 20))
 (segment (start 64.135 24.13) (end 64.135 22.225) (width 0.254) (layer B.Cu) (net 15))
 (segment (start 64.135 22.225) (end 63.5 21.59) (width 0.254) (layer B.Cu) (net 15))
 (segment (start 67.31 27.305) (end 64.135 24.13) (width 0.254) (layer B.Cu) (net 15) (status 10))
 (segment (start 63.5 21.59) (end 57.785 21.59) (width 0.254) (layer B.Cu) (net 15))
 (segment (start 69.85 27.305) (end 67.31 27.305) (width 0.254) (layer B.Cu) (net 15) (status 30))
 (via (at 57.785 21.59) (size 0.889) (layers F.Cu B.Cu) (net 15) (status 30))
 (segment (start 57.785 21.59) (end 57.4675 21.59) (width 0.254) (layer F.Cu) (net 15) (status 30))
 (segment (start 64.1096 24.7396) (end 62.23 22.86) (width 0.254) (layer F.Cu) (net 14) (status 20))
 (segment (start 64.1096 31.2928) (end 64.1096 24.7396) (width 0.254) (layer F.Cu) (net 14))
 (segment (start 61.5696 33.8328) (end 64.1096 31.2928) (width 0.254) (layer F.Cu) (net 14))
 (segment (start 35.1028 33.8328) (end 61.5696 33.8328) (width 0.254) (layer F.Cu) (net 14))
 (segment (start 34.5948 33.3248) (end 35.1028 33.8328) (width 0.254) (layer F.Cu) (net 14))
 (segment (start 34.5948 30.2768) (end 34.5948 33.3248) (width 0.254) (layer F.Cu) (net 14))
 (segment (start 36.195 29.21) (end 35.6616 29.21) (width 0.254) (layer F.Cu) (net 14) (status 30))
 (segment (start 35.6616 29.21) (end 34.5948 30.2768) (width 0.254) (layer F.Cu) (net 14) (status 10))
 (segment (start 36.195 24.13) (end 34.8742 24.13) (width 0.381) (layer F.Cu) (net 11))
 (segment (start 25.6413 24.765) (end 24.765 24.765) (width 0.381) (layer F.Cu) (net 11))
 (segment (start 27.7368 26.8605) (end 25.6413 24.765) (width 0.381) (layer F.Cu) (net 11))
 (via (at 27.7368 26.8605) (size 0.889) (layers F.Cu B.Cu) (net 11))
 (segment (start 27.7368 23.0886) (end 27.7368 26.8605) (width 0.381) (layer B.Cu) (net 11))
 (segment (start 27.8511 22.9743) (end 27.7368 23.0886) (width 0.381) (layer B.Cu) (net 11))
 (via (at 27.8511 22.9743) (size 0.889) (layers F.Cu B.Cu) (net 11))
 (segment (start 33.7185 22.9743) (end 27.8511 22.9743) (width 0.381) (layer F.Cu) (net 11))
 (segment (start 34.8742 24.13) (end 33.7185 22.9743) (width 0.381) (layer F.Cu) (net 11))
 (segment (start 39.0144 17.2212) (end 39.0144 17.5006) (width 0.254) (layer F.Cu) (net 8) (status 30))
 (segment (start 39.0144 17.5006) (end 36.195 20.32) (width 0.254) (layer F.Cu) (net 8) (status 30))
 (segment (start 21.1836 29.5148) (end 21.1836 30.48) (width 0.254) (layer F.Cu) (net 16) (status 10))
 (segment (start 65.1256 26.9494) (end 67.31 24.765) (width 0.254) (layer F.Cu) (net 16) (status 20))
 (segment (start 65.1256 31.2928) (end 65.1256 26.9494) (width 0.254) (layer F.Cu) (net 16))
 (segment (start 61.976 34.4424) (end 65.1256 31.2928) (width 0.254) (layer F.Cu) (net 16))
 (segment (start 25.146 34.4424) (end 61.976 34.4424) (width 0.254) (layer F.Cu) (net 16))
 (segment (start 21.1836 30.48) (end 25.146 34.4424) (width 0.254) (layer F.Cu) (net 16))
 (segment (start 69.85 24.765) (end 67.31 24.765) (width 0.254) (layer B.Cu) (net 16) (status 30))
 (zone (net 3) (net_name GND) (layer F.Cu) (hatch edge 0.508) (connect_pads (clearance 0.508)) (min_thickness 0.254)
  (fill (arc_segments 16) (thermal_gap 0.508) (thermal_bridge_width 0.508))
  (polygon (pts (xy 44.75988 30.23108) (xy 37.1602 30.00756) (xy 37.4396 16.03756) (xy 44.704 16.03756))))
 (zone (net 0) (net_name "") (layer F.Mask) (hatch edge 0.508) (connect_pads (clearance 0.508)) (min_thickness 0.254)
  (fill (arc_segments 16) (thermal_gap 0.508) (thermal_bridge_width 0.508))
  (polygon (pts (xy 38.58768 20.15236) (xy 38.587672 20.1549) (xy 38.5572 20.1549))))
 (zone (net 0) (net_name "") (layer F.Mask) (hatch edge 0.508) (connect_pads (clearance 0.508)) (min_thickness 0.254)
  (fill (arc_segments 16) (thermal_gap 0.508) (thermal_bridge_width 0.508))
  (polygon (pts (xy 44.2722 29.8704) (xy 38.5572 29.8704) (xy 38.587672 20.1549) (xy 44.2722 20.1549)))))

